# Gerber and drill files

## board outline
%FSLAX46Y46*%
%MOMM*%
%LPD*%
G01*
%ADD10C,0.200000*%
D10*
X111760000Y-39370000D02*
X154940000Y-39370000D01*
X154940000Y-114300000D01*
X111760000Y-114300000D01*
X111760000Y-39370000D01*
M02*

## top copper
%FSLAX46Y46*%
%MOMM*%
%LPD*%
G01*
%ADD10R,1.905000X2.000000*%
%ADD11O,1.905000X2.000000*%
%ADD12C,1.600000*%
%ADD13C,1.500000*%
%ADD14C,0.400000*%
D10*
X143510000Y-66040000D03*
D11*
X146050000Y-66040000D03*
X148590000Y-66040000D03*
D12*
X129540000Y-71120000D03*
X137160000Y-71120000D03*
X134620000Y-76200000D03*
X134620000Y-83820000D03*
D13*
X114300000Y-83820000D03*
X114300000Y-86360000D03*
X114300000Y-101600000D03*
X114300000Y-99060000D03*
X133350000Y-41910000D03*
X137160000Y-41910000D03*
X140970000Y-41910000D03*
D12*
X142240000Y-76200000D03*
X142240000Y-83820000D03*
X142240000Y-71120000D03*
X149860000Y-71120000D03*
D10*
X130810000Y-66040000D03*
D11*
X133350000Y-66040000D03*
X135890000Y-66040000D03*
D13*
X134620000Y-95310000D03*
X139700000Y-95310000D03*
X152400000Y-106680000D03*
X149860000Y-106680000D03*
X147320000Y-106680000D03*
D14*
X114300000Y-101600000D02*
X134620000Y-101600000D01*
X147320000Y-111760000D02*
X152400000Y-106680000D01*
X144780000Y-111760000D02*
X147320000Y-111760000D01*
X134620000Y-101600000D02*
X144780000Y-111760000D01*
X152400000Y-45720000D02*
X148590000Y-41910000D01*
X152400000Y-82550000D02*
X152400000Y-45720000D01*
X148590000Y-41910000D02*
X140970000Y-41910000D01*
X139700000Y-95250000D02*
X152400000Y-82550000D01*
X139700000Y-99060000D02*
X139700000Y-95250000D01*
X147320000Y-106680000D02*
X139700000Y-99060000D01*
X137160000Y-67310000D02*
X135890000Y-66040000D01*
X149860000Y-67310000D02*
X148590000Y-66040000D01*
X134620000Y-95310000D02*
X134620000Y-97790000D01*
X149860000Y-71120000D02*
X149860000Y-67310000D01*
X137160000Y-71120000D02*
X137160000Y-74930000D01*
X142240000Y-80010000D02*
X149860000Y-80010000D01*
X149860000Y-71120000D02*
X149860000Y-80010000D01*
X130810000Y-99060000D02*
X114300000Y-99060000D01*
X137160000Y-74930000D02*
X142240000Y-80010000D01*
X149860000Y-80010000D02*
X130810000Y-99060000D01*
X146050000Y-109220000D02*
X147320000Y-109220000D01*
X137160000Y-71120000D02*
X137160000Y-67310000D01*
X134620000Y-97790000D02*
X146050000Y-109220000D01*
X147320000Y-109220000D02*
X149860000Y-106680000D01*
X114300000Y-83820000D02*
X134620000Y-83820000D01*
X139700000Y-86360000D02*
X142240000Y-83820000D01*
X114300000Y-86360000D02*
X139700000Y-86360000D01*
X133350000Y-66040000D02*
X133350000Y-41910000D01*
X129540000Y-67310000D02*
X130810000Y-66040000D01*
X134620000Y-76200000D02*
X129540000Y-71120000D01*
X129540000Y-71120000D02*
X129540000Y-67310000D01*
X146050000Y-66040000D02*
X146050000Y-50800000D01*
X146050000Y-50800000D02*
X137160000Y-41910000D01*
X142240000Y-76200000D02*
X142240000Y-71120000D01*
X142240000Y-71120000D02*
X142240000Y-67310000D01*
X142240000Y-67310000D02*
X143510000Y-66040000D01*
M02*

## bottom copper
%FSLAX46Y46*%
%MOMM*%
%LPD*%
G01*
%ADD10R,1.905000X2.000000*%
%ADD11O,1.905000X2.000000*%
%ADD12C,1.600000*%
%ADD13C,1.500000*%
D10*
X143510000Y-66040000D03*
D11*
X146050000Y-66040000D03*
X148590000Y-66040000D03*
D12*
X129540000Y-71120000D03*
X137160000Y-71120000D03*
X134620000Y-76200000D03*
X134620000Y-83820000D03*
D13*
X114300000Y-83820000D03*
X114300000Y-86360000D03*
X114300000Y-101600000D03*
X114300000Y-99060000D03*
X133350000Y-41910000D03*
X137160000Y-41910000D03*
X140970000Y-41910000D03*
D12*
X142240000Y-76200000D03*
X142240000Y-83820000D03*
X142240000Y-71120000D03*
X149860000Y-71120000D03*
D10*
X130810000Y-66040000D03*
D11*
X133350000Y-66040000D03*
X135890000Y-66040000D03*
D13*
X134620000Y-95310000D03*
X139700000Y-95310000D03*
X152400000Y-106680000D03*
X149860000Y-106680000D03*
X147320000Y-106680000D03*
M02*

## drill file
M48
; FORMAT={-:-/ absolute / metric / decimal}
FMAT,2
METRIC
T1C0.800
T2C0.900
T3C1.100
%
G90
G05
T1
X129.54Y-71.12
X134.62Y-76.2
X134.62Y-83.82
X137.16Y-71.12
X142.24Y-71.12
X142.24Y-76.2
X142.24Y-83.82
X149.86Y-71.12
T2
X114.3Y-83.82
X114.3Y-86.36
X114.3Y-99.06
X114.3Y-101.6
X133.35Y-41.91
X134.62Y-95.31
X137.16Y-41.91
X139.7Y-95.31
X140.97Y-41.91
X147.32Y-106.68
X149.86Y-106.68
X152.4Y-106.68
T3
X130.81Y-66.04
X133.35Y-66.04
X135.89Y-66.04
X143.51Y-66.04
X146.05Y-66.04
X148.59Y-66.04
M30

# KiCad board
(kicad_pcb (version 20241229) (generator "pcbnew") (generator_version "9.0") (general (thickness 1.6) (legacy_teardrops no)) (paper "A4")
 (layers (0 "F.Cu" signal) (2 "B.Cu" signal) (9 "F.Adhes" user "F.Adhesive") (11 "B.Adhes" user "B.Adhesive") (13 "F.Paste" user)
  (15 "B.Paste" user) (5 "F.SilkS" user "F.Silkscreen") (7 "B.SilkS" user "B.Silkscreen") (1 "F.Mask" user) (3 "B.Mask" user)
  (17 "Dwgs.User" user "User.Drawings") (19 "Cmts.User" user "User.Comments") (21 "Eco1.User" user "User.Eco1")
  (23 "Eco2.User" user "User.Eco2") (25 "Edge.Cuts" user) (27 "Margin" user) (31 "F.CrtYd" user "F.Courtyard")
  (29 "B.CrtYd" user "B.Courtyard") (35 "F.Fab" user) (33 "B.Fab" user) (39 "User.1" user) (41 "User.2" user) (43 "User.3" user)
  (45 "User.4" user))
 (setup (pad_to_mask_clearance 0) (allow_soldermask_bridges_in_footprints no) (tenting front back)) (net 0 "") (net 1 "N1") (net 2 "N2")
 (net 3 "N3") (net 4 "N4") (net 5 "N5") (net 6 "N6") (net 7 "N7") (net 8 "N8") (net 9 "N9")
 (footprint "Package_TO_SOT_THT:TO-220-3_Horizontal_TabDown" (layer "F.Cu") (at 143.51 66.04)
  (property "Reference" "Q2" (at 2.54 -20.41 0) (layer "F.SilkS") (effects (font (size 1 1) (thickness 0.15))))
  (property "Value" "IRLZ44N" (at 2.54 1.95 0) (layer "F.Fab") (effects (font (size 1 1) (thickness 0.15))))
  (pad "1" thru_hole rect (at 0 0) (size 1.905 2) (drill 1.1) (layers "*.Cu" "*.Mask") (remove_unused_layers no) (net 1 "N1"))
  (pad "2" thru_hole oval (at 2.54 0) (size 1.905 2) (drill 1.1) (layers "*.Cu" "*.Mask") (remove_unused_layers no) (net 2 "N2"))
  (pad "3" thru_hole oval (at 5.08 0) (size 1.905 2) (drill 1.1) (layers "*.Cu" "*.Mask") (remove_unused_layers no) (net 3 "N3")))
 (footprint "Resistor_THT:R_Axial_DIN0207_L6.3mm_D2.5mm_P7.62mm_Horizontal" (layer "F.Cu") (at 129.54 71.12)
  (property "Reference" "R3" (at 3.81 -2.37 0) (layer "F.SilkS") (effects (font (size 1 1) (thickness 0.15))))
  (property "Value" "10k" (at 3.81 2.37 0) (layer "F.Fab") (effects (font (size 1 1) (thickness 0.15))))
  (pad "1" thru_hole circle (at 0 0) (size 1.6 1.6) (drill 0.8) (layers "*.Cu" "*.Mask") (remove_unused_layers no) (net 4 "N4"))
  (pad "2" thru_hole circle (at 7.62 0) (size 1.6 1.6) (drill 0.8) (layers "*.Cu" "*.Mask") (remove_unused_layers no) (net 3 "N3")))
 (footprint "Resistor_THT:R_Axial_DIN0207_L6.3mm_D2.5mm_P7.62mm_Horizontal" (layer "F.Cu") (at 134.62 76.2 -90)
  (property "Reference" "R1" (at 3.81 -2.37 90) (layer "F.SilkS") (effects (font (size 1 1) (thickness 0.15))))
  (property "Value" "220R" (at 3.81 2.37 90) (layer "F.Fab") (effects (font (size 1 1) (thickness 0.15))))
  (pad "1" thru_hole circle (at 0 0 270) (size 1.6 1.6) (drill 0.8) (layers "*.Cu" "*.Mask") (remove_unused_layers no) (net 4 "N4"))
  (pad "2" thru_hole circle (at 7.62 0 270) (size 1.6 1.6) (drill 0.8) (layers "*.Cu" "*.Mask") (remove_unused_layers no) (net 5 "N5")))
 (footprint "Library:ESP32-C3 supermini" (layer "F.Cu") (at 121.92 91.44)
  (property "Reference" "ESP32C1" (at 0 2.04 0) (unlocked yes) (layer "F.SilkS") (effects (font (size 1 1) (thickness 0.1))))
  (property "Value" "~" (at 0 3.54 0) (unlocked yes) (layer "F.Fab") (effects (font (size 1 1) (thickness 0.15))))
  (pad "0" thru_hole circle (at -7.62 -7.62) (size 1.5 1.5) (drill 0.9) (layers "*.Cu" "*.Mask") (remove_unused_layers yes)
   (keep_end_layers yes) (zone_layer_connections) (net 5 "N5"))
  (pad "1" thru_hole circle (at -7.62 -5.08) (size 1.5 1.5) (drill 0.9) (layers "*.Cu" "*.Mask") (remove_unused_layers yes)
   (keep_end_layers yes) (zone_layer_connections) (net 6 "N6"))
  (pad "5V" thru_hole circle (at -7.62 10.16) (size 1.5 1.5) (drill 0.9) (layers "*.Cu" "*.Mask") (remove_unused_layers yes)
   (keep_end_layers yes) (zone_layer_connections) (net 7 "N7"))
  (pad "GND" thru_hole circle (at -7.62 7.62) (size 1.5 1.5) (drill 0.9) (layers "*.Cu" "*.Mask") (remove_unused_layers yes)
   (keep_end_layers yes) (zone_layer_connections) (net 3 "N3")))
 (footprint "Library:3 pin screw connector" (layer "F.Cu") (at 137.16 41.91)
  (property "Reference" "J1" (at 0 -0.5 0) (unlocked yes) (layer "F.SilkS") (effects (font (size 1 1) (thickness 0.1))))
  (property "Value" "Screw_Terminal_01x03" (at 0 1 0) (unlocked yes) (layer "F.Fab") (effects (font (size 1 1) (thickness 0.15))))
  (pad "1" thru_hole circle (at -3.81 0) (size 1.5 1.5) (drill 0.9) (layers "*.Cu" "*.Mask") (remove_unused_layers yes)
   (keep_end_layers yes) (zone_layer_connections) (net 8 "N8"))
  (pad "2" thru_hole circle (at 0 0) (size 1.5 1.5) (drill 0.9) (layers "*.Cu" "*.Mask") (remove_unused_layers yes) (keep_end_layers yes)
   (zone_layer_connections) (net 2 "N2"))
  (pad "3" thru_hole circle (at 3.81 0) (size 1.5 1.5) (drill 0.9) (layers "*.Cu" "*.Mask") (remove_unused_layers yes) (keep_end_layers yes)
   (zone_layer_connections) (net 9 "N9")))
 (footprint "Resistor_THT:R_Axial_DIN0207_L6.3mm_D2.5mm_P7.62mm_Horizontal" (layer "F.Cu") (at 142.24 76.2 -90)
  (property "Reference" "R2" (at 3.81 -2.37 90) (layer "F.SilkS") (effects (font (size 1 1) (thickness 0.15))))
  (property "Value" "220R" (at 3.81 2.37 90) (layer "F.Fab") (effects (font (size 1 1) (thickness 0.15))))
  (pad "1" thru_hole circle (at 0 0 270) (size 1.6 1.6) (drill 0.8) (layers "*.Cu" "*.Mask") (remove_unused_layers no) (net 1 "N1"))
  (pad "2" thru_hole circle (at 7.62 0 270) (size 1.6 1.6) (drill 0.8) (layers "*.Cu" "*.Mask") (remove_unused_layers no) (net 6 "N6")))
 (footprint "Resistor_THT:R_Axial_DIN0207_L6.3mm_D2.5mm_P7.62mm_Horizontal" (layer "F.Cu") (at 142.24 71.12)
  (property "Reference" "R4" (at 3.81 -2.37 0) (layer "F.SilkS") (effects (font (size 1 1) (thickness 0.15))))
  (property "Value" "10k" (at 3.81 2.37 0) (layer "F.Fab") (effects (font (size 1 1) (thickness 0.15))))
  (pad "1" thru_hole circle (at 0 0) (size 1.6 1.6) (drill 0.8) (layers "*.Cu" "*.Mask") (remove_unused_layers no) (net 1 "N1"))
  (pad "2" thru_hole circle (at 7.62 0) (size 1.6 1.6) (drill 0.8) (layers "*.Cu" "*.Mask") (remove_unused_layers no) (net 3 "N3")))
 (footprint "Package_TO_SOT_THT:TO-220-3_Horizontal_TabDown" (layer "F.Cu") (at 130.81 66.04)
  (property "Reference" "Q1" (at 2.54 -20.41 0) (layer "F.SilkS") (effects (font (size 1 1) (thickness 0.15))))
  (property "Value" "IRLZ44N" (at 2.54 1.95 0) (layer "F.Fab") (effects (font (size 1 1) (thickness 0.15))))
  (pad "1" thru_hole rect (at 0 0) (size 1.905 2) (drill 1.1) (layers "*.Cu" "*.Mask") (remove_unused_layers no) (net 4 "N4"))
  (pad "2" thru_hole oval (at 2.54 0) (size 1.905 2) (drill 1.1) (layers "*.Cu" "*.Mask") (remove_unused_layers no) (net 8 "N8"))
  (pad "3" thru_hole oval (at 5.08 0) (size 1.905 2) (drill 1.1) (layers "*.Cu" "*.Mask") (remove_unused_layers no) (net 3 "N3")))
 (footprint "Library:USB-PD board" (layer "F.Cu") (at 137.16 97.85)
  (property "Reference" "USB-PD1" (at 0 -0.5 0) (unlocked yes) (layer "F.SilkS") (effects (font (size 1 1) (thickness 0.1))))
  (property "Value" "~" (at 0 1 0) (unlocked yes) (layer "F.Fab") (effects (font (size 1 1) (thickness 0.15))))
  (pad "GND" thru_hole circle (at -2.54 -2.54) (size 1.5 1.5) (drill 0.9) (layers "*.Cu" "*.Mask") (remove_unused_layers yes)
   (keep_end_layers yes) (zone_layer_connections) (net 3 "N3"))
  (pad "VBUS" thru_hole circle (at 2.54 -2.54) (size 1.5 1.5) (drill 0.9) (layers "*.Cu" "*.Mask") (remove_unused_layers yes)
   (keep_end_layers yes) (zone_layer_connections) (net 9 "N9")))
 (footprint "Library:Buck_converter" (layer "F.Cu") (at 148.59 111.76 180)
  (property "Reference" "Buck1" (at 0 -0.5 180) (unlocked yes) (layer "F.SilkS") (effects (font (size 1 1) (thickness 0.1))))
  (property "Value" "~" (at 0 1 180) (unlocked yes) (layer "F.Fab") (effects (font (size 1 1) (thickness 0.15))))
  (pad "1" thru_hole circle (at -3.81 5.08 180) (size 1.5 1.5) (drill 0.9) (layers "*.Cu" "*.Mask") (remove_unused_layers yes)
   (keep_end_layers yes) (zone_layer_connections) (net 7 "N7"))
  (pad "2" thru_hole circle (at -1.27 5.08 180) (size 1.5 1.5) (drill 0.9) (layers "*.Cu" "*.Mask") (remove_unused_layers yes)
   (keep_end_layers yes) (zone_layer_connections) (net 3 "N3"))
  (pad "3" thru_hole circle (at 1.27 5.08 180) (size 1.5 1.5) (drill 0.9) (layers "*.Cu" "*.Mask") (remove_unused_layers yes)
   (keep_end_layers yes) (zone_layer_connections) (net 9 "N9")))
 (gr_rect (start 111.76 39.37) (end 154.94 114.3) (stroke (width 0.2) (type solid)) (fill no) (layer "Edge.Cuts"))
 (segment (start 114.3 101.6) (end 134.62 101.6) (width 0.4) (layer "F.Cu") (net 7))
 (segment (start 147.32 111.76) (end 152.4 106.68) (width 0.4) (layer "F.Cu") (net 7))
 (segment (start 144.78 111.76) (end 147.32 111.76) (width 0.4) (layer "F.Cu") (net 7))
 (segment (start 134.62 101.6) (end 144.78 111.76) (width 0.4) (layer "F.Cu") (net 7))
 (segment (start 152.4 45.72) (end 148.59 41.91) (width 0.4) (layer "F.Cu") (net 9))
 (segment (start 152.4 82.55) (end 152.4 45.72) (width 0.4) (layer "F.Cu") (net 9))
 (segment (start 148.59 41.91) (end 140.97 41.91) (width 0.4) (layer "F.Cu") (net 9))
 (segment (start 139.7 95.25) (end 152.4 82.55) (width 0.4) (layer "F.Cu") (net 9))
 (segment (start 139.7 99.06) (end 139.7 95.25) (width 0.4) (layer "F.Cu") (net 9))
 (segment (start 147.32 106.68) (end 139.7 99.06) (width 0.4) (layer "F.Cu") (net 9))
 (segment (start 137.16 67.31) (end 135.89 66.04) (width 0.4) (layer "F.Cu") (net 3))
 (segment (start 149.86 67.31) (end 148.59 66.04) (width 0.4) (layer "F.Cu") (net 3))
 (segment (start 134.62 95.31) (end 134.62 97.79) (width 0.4) (layer "F.Cu") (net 3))
 (segment (start 149.86 71.12) (end 149.86 67.31) (width 0.4) (layer "F.Cu") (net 3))
 (segment (start 137.16 71.12) (end 137.16 74.93) (width 0.4) (layer "F.Cu") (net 3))
 (segment (start 142.24 80.01) (end 149.86 80.01) (width 0.4) (layer "F.Cu") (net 3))
 (segment (start 149.86 71.12) (end 149.86 80.01) (width 0.4) (layer "F.Cu") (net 3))
 (segment (start 130.81 99.06) (end 114.3 99.06) (width 0.4) (layer "F.Cu") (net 3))
 (segment (start 137.16 74.93) (end 142.24 80.01) (width 0.4) (layer "F.Cu") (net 3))
 (segment (start 149.86 80.01) (end 130.81 99.06) (width 0.4) (layer "F.Cu") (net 3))
 (segment (start 146.05 109.22) (end 147.32 109.22) (width 0.4) (layer "F.Cu") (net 3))
 (segment (start 137.16 71.12) (end 137.16 67.31) (width 0.4) (layer "F.Cu") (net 3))
 (segment (start 134.62 97.79) (end 146.05 109.22) (width 0.4) (layer "F.Cu") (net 3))
 (segment (start 147.32 109.22) (end 149.86 106.68) (width 0.4) (layer "F.Cu") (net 3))
 (segment (start 114.3 83.82) (end 134.62 83.82) (width 0.4) (layer "F.Cu") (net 5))
 (segment (start 139.7 86.36) (end 142.24 83.82) (width 0.4) (layer "F.Cu") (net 6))
 (segment (start 114.3 86.36) (end 139.7 86.36) (width 0.4) (layer "F.Cu") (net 6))
 (segment (start 133.35 66.04) (end 133.35 41.91) (width 0.4) (layer "F.Cu") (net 8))
 (segment (start 129.54 67.31) (end 130.81 66.04) (width 0.4) (layer "F.Cu") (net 4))
 (segment (start 134.62 76.2) (end 129.54 71.12) (width 0.4) (layer "F.Cu") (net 4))
 (segment (start 129.54 71.12) (end 129.54 67.31) (width 0.4) (layer "F.Cu") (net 4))
 (segment (start 146.05 66.04) (end 146.05 50.8) (width 0.4) (layer "F.Cu") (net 2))
 (segment (start 146.05 50.8) (end 137.16 41.91) (width 0.4) (layer "F.Cu") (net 2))
 (segment (start 142.24 76.2) (end 142.24 71.12) (width 0.4) (layer "F.Cu") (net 1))
 (segment (start 142.24 71.12) (end 142.24 67.31) (width 0.4) (layer "F.Cu") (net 1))
 (segment (start 142.24 67.31) (end 143.51 66.04) (width 0.4) (layer "F.Cu") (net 1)))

